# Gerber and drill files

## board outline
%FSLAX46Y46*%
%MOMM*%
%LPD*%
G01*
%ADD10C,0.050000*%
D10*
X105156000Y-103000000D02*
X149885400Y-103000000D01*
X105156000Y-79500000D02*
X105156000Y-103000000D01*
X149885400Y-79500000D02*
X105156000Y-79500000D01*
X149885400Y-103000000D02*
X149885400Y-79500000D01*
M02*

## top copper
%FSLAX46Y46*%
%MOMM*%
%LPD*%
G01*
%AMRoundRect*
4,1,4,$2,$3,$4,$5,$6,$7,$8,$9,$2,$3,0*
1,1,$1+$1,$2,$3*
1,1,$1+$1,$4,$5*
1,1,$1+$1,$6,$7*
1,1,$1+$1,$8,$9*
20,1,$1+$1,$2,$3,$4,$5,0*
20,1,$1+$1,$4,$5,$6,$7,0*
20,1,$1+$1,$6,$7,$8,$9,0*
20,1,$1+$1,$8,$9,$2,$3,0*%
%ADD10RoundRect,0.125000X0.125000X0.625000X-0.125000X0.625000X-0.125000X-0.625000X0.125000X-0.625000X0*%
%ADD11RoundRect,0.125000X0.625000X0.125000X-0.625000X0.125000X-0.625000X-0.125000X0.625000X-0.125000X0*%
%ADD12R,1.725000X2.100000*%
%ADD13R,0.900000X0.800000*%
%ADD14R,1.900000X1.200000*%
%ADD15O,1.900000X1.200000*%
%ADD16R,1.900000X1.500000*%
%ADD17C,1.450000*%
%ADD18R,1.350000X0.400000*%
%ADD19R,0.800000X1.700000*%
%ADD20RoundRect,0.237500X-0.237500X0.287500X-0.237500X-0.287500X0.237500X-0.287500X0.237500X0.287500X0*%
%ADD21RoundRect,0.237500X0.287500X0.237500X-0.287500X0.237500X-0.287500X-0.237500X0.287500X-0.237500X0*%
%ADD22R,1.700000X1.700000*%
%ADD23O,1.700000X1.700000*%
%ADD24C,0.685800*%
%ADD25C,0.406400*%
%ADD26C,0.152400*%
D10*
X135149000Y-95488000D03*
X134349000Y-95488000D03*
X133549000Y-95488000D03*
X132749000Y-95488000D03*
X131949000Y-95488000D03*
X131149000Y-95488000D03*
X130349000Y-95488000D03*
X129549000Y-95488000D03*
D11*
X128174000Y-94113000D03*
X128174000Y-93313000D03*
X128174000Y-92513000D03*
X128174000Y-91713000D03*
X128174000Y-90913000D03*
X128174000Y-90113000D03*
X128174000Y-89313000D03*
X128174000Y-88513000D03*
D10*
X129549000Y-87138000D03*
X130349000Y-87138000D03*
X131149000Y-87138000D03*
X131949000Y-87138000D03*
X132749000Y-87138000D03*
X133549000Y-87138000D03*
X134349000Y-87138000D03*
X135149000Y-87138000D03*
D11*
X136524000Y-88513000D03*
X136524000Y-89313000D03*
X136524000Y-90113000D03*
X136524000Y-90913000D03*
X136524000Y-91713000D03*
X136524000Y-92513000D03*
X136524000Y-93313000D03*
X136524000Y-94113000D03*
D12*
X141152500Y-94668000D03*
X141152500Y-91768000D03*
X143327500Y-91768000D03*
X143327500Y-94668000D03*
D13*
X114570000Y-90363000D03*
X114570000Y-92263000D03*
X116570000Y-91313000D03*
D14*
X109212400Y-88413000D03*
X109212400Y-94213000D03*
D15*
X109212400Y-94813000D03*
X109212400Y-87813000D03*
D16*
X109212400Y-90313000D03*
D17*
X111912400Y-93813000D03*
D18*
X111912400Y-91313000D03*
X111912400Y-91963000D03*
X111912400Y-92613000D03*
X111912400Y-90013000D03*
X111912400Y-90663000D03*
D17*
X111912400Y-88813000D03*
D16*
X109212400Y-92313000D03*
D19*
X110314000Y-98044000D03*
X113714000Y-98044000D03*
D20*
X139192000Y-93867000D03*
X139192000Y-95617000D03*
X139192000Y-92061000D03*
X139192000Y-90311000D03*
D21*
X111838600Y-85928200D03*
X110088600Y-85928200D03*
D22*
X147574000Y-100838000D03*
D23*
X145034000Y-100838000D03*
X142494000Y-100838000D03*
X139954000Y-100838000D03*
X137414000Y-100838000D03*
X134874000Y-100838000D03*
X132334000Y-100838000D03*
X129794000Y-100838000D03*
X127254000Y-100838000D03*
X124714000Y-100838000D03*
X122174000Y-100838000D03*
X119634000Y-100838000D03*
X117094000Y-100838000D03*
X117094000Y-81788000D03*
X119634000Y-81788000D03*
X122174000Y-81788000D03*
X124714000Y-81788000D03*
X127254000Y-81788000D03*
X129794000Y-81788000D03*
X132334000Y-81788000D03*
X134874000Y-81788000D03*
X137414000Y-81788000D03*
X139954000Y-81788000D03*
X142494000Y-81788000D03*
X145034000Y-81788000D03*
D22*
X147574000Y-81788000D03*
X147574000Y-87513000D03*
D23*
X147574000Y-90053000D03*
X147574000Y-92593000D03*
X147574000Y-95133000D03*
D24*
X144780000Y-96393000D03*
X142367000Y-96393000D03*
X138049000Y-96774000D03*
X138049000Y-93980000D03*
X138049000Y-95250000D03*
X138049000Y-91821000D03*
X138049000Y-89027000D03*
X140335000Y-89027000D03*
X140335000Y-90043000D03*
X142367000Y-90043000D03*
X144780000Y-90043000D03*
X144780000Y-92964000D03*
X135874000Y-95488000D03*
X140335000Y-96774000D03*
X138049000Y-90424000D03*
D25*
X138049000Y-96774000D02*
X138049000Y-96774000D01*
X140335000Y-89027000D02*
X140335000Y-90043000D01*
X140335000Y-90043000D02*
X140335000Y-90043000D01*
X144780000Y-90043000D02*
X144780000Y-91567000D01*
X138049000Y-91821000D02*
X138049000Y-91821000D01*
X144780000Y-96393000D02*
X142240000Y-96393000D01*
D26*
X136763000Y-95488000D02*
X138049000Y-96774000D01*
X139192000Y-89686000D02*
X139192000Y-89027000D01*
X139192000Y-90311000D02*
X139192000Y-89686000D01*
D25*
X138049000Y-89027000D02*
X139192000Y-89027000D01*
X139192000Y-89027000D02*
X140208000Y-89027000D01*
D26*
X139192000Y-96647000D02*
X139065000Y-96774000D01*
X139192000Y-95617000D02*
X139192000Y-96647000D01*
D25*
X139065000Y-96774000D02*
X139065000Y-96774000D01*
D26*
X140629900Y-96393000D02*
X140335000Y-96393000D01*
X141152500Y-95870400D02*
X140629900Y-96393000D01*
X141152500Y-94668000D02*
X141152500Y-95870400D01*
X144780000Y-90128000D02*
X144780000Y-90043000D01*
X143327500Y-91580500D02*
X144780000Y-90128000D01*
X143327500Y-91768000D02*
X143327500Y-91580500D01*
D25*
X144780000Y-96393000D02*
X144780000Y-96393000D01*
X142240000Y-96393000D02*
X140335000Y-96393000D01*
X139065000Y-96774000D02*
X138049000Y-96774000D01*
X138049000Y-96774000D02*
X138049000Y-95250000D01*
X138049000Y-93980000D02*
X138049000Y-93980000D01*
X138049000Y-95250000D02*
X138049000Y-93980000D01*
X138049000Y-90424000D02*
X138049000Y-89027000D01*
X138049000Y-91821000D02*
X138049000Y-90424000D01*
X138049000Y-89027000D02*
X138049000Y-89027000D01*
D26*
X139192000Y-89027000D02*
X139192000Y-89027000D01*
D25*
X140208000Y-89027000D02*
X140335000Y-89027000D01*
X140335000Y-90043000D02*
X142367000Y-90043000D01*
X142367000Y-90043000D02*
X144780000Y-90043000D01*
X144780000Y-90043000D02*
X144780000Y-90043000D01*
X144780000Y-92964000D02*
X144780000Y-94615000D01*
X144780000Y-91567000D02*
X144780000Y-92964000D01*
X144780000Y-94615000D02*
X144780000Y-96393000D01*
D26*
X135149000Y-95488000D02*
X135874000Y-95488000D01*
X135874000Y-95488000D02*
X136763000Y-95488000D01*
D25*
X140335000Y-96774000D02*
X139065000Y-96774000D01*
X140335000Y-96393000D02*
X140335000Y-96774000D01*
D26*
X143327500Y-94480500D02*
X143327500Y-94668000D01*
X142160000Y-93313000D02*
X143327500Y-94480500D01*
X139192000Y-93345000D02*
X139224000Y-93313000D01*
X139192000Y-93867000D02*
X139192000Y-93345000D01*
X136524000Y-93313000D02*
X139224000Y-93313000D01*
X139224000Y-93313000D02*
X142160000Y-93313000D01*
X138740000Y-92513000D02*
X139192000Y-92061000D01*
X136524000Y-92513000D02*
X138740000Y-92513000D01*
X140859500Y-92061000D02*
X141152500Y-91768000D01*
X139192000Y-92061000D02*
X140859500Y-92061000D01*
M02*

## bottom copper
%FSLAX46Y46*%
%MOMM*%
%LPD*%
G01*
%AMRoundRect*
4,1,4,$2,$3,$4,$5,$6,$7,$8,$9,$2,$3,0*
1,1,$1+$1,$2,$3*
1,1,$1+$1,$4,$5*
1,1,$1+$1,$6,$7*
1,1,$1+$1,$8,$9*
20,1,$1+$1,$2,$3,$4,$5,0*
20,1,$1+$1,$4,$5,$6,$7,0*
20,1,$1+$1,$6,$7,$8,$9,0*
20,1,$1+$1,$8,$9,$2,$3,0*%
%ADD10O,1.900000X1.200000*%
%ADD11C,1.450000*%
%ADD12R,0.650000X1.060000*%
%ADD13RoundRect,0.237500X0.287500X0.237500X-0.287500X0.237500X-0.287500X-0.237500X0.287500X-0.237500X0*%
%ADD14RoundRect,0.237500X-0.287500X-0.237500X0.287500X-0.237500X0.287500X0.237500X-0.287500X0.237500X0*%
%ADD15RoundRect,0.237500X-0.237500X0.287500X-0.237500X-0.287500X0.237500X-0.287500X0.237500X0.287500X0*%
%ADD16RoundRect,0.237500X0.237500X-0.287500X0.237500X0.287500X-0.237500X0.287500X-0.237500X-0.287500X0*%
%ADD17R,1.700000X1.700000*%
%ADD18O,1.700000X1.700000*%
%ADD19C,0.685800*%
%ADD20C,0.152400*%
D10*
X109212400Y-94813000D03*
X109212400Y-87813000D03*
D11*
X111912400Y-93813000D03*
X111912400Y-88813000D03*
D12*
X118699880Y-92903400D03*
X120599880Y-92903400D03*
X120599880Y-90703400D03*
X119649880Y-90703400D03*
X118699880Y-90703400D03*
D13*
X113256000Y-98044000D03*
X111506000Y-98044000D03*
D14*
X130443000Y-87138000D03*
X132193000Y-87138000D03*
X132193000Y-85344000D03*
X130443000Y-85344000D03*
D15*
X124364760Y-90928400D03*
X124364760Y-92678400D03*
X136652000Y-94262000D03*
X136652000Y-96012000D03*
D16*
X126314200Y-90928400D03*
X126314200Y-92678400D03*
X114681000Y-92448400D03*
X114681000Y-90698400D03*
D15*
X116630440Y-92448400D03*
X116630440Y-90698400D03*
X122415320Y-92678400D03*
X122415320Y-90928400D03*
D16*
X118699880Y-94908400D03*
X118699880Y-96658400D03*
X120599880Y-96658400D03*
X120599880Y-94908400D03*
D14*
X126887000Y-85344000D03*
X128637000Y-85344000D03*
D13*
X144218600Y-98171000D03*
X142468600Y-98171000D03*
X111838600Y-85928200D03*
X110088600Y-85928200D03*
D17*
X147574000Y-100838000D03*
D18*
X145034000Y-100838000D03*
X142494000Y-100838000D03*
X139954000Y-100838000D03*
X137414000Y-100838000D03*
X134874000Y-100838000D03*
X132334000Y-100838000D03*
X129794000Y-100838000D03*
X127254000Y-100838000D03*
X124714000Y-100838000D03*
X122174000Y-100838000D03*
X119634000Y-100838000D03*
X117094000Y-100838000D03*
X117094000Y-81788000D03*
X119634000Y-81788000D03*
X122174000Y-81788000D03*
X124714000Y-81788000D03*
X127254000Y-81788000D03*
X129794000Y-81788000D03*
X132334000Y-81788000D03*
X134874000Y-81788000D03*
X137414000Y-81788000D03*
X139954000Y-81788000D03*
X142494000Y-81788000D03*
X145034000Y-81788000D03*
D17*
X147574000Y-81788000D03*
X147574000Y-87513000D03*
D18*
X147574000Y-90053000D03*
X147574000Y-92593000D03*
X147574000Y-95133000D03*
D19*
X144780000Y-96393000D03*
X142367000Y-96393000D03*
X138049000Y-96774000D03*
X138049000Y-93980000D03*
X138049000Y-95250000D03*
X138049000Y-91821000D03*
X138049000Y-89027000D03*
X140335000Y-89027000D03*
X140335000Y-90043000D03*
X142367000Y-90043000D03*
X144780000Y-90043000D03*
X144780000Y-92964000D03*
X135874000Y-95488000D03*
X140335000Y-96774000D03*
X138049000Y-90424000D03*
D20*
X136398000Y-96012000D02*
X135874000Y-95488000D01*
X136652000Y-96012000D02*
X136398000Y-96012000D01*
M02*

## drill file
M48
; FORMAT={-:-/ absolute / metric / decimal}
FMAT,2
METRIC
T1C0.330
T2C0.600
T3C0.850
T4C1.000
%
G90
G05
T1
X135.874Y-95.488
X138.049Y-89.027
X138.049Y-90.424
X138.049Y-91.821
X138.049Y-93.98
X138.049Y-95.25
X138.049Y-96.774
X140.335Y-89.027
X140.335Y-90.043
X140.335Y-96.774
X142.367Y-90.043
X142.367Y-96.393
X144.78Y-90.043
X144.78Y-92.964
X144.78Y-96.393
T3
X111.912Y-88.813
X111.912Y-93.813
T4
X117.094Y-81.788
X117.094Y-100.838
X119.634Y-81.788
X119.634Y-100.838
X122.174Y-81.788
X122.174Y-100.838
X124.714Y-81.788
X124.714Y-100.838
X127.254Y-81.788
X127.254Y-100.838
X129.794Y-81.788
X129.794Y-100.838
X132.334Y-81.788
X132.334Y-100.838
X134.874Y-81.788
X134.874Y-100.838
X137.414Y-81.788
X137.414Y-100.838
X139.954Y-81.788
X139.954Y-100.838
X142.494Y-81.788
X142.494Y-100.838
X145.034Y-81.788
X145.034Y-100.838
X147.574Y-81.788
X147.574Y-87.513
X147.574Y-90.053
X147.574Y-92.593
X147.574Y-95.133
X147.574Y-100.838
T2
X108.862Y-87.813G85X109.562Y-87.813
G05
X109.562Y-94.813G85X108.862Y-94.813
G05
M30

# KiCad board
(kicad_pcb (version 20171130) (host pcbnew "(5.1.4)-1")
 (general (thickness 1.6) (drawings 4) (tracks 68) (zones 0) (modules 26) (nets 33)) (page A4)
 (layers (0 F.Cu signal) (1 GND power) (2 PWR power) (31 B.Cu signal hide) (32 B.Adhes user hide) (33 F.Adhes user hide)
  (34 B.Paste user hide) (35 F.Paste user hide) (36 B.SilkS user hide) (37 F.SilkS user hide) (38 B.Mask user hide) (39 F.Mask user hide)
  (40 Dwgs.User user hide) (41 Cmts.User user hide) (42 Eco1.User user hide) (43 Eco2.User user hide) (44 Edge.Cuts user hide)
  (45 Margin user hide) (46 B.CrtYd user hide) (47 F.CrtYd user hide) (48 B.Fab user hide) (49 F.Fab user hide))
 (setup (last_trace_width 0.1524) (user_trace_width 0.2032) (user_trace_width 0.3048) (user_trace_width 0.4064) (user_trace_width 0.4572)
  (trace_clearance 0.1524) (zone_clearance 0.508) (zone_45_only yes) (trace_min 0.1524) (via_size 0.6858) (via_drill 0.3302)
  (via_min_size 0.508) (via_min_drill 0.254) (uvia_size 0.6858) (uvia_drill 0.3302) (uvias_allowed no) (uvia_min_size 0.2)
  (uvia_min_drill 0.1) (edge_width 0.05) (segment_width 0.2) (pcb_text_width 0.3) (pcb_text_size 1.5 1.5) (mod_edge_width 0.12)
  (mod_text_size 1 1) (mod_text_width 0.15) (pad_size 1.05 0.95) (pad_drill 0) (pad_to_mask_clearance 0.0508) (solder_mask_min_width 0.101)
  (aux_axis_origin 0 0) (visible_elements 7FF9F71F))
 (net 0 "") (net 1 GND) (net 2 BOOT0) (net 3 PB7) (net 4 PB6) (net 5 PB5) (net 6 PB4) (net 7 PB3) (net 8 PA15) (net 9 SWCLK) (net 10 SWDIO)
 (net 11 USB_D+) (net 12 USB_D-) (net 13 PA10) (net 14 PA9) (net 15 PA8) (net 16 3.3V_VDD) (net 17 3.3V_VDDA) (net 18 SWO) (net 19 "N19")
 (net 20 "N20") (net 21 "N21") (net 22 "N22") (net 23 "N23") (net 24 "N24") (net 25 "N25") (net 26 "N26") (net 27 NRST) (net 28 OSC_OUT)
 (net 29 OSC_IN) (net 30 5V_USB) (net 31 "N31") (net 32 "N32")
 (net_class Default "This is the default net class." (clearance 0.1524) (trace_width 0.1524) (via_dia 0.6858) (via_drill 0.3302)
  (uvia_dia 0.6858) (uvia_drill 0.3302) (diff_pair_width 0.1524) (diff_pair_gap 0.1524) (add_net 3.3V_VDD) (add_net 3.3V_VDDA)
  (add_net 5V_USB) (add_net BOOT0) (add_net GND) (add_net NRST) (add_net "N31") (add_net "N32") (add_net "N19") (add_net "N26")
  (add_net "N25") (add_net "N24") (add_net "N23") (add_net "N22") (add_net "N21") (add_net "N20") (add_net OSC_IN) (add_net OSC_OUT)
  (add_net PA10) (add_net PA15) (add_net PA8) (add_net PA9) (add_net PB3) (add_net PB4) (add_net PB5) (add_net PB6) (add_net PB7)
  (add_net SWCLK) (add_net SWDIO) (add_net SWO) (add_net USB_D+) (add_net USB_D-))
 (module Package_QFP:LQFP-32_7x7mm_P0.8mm (layer F.Cu) (at 132.349 91.313 180)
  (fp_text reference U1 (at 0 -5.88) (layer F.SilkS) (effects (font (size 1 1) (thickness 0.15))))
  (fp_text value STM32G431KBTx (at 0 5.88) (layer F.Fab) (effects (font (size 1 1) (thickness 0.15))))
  (pad 32 smd roundrect (at -2.8 -4.175 180) (size 0.5 1.5) (layers F.Cu F.Paste F.Mask) (roundrect_rratio 0.25) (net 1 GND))
  (pad 31 smd roundrect (at -2 -4.175 180) (size 0.5 1.5) (layers F.Cu F.Paste F.Mask) (roundrect_rratio 0.25) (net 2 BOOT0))
  (pad 30 smd roundrect (at -1.2 -4.175 180) (size 0.5 1.5) (layers F.Cu F.Paste F.Mask) (roundrect_rratio 0.25) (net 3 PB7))
  (pad 29 smd roundrect (at -0.4 -4.175 180) (size 0.5 1.5) (layers F.Cu F.Paste F.Mask) (roundrect_rratio 0.25) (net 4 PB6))
  (pad 28 smd roundrect (at 0.4 -4.175 180) (size 0.5 1.5) (layers F.Cu F.Paste F.Mask) (roundrect_rratio 0.25) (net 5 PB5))
  (pad 27 smd roundrect (at 1.2 -4.175 180) (size 0.5 1.5) (layers F.Cu F.Paste F.Mask) (roundrect_rratio 0.25) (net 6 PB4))
  (pad 26 smd roundrect (at 2 -4.175 180) (size 0.5 1.5) (layers F.Cu F.Paste F.Mask) (roundrect_rratio 0.25) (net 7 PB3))
  (pad 25 smd roundrect (at 2.8 -4.175 180) (size 0.5 1.5) (layers F.Cu F.Paste F.Mask) (roundrect_rratio 0.25) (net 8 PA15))
  (pad 24 smd roundrect (at 4.175 -2.8 180) (size 1.5 0.5) (layers F.Cu F.Paste F.Mask) (roundrect_rratio 0.25) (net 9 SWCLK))
  (pad 23 smd roundrect (at 4.175 -2 180) (size 1.5 0.5) (layers F.Cu F.Paste F.Mask) (roundrect_rratio 0.25) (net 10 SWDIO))
  (pad 22 smd roundrect (at 4.175 -1.2 180) (size 1.5 0.5) (layers F.Cu F.Paste F.Mask) (roundrect_rratio 0.25) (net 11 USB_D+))
  (pad 21 smd roundrect (at 4.175 -0.4 180) (size 1.5 0.5) (layers F.Cu F.Paste F.Mask) (roundrect_rratio 0.25) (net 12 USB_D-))
  (pad 20 smd roundrect (at 4.175 0.4 180) (size 1.5 0.5) (layers F.Cu F.Paste F.Mask) (roundrect_rratio 0.25) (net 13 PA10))
  (pad 19 smd roundrect (at 4.175 1.2 180) (size 1.5 0.5) (layers F.Cu F.Paste F.Mask) (roundrect_rratio 0.25) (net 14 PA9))
  (pad 18 smd roundrect (at 4.175 2 180) (size 1.5 0.5) (layers F.Cu F.Paste F.Mask) (roundrect_rratio 0.25) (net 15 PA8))
  (pad 17 smd roundrect (at 4.175 2.8 180) (size 1.5 0.5) (layers F.Cu F.Paste F.Mask) (roundrect_rratio 0.25) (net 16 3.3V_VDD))
  (pad 16 smd roundrect (at 2.8 4.175 180) (size 0.5 1.5) (layers F.Cu F.Paste F.Mask) (roundrect_rratio 0.25) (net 1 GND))
  (pad 15 smd roundrect (at 2 4.175 180) (size 0.5 1.5) (layers F.Cu F.Paste F.Mask) (roundrect_rratio 0.25) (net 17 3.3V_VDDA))
  (pad 14 smd roundrect (at 1.2 4.175 180) (size 0.5 1.5) (layers F.Cu F.Paste F.Mask) (roundrect_rratio 0.25) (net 1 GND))
  (pad 13 smd roundrect (at 0.4 4.175 180) (size 0.5 1.5) (layers F.Cu F.Paste F.Mask) (roundrect_rratio 0.25) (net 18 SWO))
  (pad 12 smd roundrect (at -0.4 4.175 180) (size 0.5 1.5) (layers F.Cu F.Paste F.Mask) (roundrect_rratio 0.25) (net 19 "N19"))
  (pad 11 smd roundrect (at -1.2 4.175 180) (size 0.5 1.5) (layers F.Cu F.Paste F.Mask) (roundrect_rratio 0.25) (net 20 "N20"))
  (pad 10 smd roundrect (at -2 4.175 180) (size 0.5 1.5) (layers F.Cu F.Paste F.Mask) (roundrect_rratio 0.25) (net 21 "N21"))
  (pad 9 smd roundrect (at -2.8 4.175 180) (size 0.5 1.5) (layers F.Cu F.Paste F.Mask) (roundrect_rratio 0.25) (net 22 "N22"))
  (pad 8 smd roundrect (at -4.175 2.8 180) (size 1.5 0.5) (layers F.Cu F.Paste F.Mask) (roundrect_rratio 0.25) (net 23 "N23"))
  (pad 7 smd roundrect (at -4.175 2 180) (size 1.5 0.5) (layers F.Cu F.Paste F.Mask) (roundrect_rratio 0.25) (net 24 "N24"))
  (pad 6 smd roundrect (at -4.175 1.2 180) (size 1.5 0.5) (layers F.Cu F.Paste F.Mask) (roundrect_rratio 0.25) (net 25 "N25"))
  (pad 5 smd roundrect (at -4.175 0.4 180) (size 1.5 0.5) (layers F.Cu F.Paste F.Mask) (roundrect_rratio 0.25) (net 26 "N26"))
  (pad 4 smd roundrect (at -4.175 -0.4 180) (size 1.5 0.5) (layers F.Cu F.Paste F.Mask) (roundrect_rratio 0.25) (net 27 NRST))
  (pad 3 smd roundrect (at -4.175 -1.2 180) (size 1.5 0.5) (layers F.Cu F.Paste F.Mask) (roundrect_rratio 0.25) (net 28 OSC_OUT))
  (pad 2 smd roundrect (at -4.175 -2 180) (size 1.5 0.5) (layers F.Cu F.Paste F.Mask) (roundrect_rratio 0.25) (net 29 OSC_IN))
  (pad 1 smd roundrect (at -4.175 -2.8 180) (size 1.5 0.5) (layers F.Cu F.Paste F.Mask) (roundrect_rratio 0.25) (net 16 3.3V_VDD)))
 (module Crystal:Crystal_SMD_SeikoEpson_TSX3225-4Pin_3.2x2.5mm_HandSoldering (layer F.Cu) (at 142.24 93.218 90)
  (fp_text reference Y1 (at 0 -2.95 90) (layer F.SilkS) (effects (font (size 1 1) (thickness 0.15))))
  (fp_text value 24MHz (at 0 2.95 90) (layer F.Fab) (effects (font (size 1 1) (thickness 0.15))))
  (pad 4 smd rect (at -1.45 -1.0875 90) (size 2.1 1.725) (layers F.Cu F.Paste F.Mask) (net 1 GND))
  (pad 3 smd rect (at 1.45 -1.0875 90) (size 2.1 1.725) (layers F.Cu F.Paste F.Mask) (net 28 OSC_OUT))
  (pad 2 smd rect (at 1.45 1.0875 90) (size 2.1 1.725) (layers F.Cu F.Paste F.Mask) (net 1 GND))
  (pad 1 smd rect (at -1.45 1.0875 90) (size 2.1 1.725) (layers F.Cu F.Paste F.Mask) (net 29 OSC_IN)))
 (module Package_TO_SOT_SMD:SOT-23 (layer F.Cu) (at 115.57 91.313)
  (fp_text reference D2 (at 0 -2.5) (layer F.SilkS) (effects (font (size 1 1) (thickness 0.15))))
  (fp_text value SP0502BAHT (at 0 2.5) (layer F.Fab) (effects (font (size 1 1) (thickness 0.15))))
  (pad 1 smd rect (at -1 -0.95) (size 0.9 0.8) (layers F.Cu F.Paste F.Mask) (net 12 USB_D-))
  (pad 2 smd rect (at -1 0.95) (size 0.9 0.8) (layers F.Cu F.Paste F.Mask) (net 11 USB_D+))
  (pad 3 smd rect (at 1 0) (size 0.9 0.8) (layers F.Cu F.Paste F.Mask) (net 1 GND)))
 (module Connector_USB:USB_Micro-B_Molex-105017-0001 (layer F.Cu) (at 110.4499 91.313 270)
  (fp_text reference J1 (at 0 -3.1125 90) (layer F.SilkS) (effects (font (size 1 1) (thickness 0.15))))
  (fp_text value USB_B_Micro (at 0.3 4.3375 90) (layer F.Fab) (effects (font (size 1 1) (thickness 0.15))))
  (pad 6 smd rect (at -2.9 1.2375 270) (size 1.2 1.9) (layers F.Cu F.Mask) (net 1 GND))
  (pad 6 smd rect (at 2.9 1.2375 270) (size 1.2 1.9) (layers F.Cu F.Mask) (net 1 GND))
  (pad 6 thru_hole oval (at 3.5 1.2375 270) (size 1.2 1.9) (drill oval 0.6 1.3) (layers *.Cu *.Mask) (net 1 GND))
  (pad 6 thru_hole oval (at -3.5 1.2375 90) (size 1.2 1.9) (drill oval 0.6 1.3) (layers *.Cu *.Mask) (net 1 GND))
  (pad 6 smd rect (at -1 1.2375 270) (size 1.5 1.9) (layers F.Cu F.Paste F.Mask) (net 1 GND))
  (pad 6 thru_hole circle (at 2.5 -1.4625 270) (size 1.45 1.45) (drill 0.85) (layers *.Cu *.Mask) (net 1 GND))
  (pad 3 smd rect (at 0 -1.4625 270) (size 0.4 1.35) (layers F.Cu F.Paste F.Mask) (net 11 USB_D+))
  (pad 4 smd rect (at 0.65 -1.4625 270) (size 0.4 1.35) (layers F.Cu F.Paste F.Mask))
  (pad 5 smd rect (at 1.3 -1.4625 270) (size 0.4 1.35) (layers F.Cu F.Paste F.Mask) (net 1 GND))
  (pad 1 smd rect (at -1.3 -1.4625 270) (size 0.4 1.35) (layers F.Cu F.Paste F.Mask) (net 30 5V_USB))
  (pad 2 smd rect (at -0.65 -1.4625 270) (size 0.4 1.35) (layers F.Cu F.Paste F.Mask) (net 12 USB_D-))
  (pad 6 thru_hole circle (at -2.5 -1.4625 270) (size 1.45 1.45) (drill 0.85) (layers *.Cu *.Mask) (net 1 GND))
  (pad 6 smd rect (at 1 1.2375 270) (size 1.5 1.9) (layers F.Cu F.Paste F.Mask) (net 1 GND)))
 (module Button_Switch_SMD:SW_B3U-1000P (layer F.Cu) (at 112.014 98.044 180)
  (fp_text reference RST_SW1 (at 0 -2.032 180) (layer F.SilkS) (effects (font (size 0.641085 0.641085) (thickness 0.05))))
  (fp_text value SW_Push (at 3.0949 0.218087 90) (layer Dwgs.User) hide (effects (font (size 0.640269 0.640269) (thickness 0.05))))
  (pad 1 smd rect (at 1.7 0 180) (size 0.8 1.7) (layers F.Cu F.Paste F.Mask) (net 1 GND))
  (pad 2 smd rect (at -1.7 0 180) (size 0.8 1.7) (layers F.Cu F.Paste F.Mask) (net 27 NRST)))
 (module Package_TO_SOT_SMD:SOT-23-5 (layer B.Cu) (at 119.64988 91.8034 270)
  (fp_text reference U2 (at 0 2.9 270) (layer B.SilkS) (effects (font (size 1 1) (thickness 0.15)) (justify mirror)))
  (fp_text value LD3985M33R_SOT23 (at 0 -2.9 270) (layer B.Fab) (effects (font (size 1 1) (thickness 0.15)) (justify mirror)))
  (pad 5 smd rect (at 1.1 0.95 270) (size 1.06 0.65) (layers B.Cu B.Paste B.Mask) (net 16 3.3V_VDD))
  (pad 4 smd rect (at 1.1 -0.95 270) (size 1.06 0.65) (layers B.Cu B.Paste B.Mask) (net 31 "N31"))
  (pad 3 smd rect (at -1.1 -0.95 270) (size 1.06 0.65) (layers B.Cu B.Paste B.Mask) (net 30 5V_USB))
  (pad 2 smd rect (at -1.1 0 270) (size 1.06 0.65) (layers B.Cu B.Paste B.Mask) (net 1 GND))
  (pad 1 smd rect (at -1.1 0.95 270) (size 1.06 0.65) (layers B.Cu B.Paste B.Mask) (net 30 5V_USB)))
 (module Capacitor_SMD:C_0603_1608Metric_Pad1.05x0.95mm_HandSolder (layer B.Cu) (at 112.381 98.044 180)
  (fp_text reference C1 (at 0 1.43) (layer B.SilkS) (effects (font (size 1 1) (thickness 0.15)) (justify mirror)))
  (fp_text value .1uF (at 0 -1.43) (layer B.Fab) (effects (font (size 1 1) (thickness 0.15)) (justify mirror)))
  (pad 1 smd roundrect (at -0.875 0 180) (size 1.05 0.95) (layers B.Cu B.Paste B.Mask) (roundrect_rratio 0.25) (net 27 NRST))
  (pad 2 smd roundrect (at 0.875 0 180) (size 1.05 0.95) (layers B.Cu B.Paste B.Mask) (roundrect_rratio 0.25) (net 1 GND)))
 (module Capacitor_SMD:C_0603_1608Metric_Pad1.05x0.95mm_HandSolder (layer F.Cu) (at 139.192 94.742 270)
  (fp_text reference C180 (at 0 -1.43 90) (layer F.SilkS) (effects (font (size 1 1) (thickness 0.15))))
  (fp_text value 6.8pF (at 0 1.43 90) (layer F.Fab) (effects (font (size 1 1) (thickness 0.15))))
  (pad 1 smd roundrect (at -0.875 0 270) (size 1.05 0.95) (layers F.Cu F.Paste F.Mask) (roundrect_rratio 0.25) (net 29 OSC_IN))
  (pad 2 smd roundrect (at 0.875 0 270) (size 1.05 0.95) (layers F.Cu F.Paste F.Mask) (roundrect_rratio 0.25) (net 1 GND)))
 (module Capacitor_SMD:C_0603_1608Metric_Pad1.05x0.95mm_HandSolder (layer F.Cu) (at 139.192 91.186 270)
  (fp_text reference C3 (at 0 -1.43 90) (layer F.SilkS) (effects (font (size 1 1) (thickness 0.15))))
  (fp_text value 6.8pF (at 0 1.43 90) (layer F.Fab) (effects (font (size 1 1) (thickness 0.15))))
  (pad 2 smd roundrect (at 0.875 0 270) (size 1.05 0.95) (layers F.Cu F.Paste F.Mask) (roundrect_rratio 0.25) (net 28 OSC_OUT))
  (pad 1 smd roundrect (at -0.875 0 270) (size 1.05 0.95) (layers F.Cu F.Paste F.Mask) (roundrect_rratio 0.25) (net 1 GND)))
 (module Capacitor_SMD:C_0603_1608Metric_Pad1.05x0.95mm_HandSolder (layer B.Cu) (at 131.318 87.138)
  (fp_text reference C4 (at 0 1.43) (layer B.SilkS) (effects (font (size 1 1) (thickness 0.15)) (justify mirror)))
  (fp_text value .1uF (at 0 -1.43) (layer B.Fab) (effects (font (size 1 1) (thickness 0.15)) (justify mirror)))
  (pad 1 smd roundrect (at -0.875 0) (size 1.05 0.95) (layers B.Cu B.Paste B.Mask) (roundrect_rratio 0.25) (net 17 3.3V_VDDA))
  (pad 2 smd roundrect (at 0.875 0) (size 1.05 0.95) (layers B.Cu B.Paste B.Mask) (roundrect_rratio 0.25) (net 1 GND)))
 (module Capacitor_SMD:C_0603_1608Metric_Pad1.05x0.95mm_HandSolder (layer B.Cu) (at 131.318 85.344)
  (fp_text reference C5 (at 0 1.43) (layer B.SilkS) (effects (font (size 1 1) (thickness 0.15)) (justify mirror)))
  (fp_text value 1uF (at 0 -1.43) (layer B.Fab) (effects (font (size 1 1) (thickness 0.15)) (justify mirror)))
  (pad 2 smd roundrect (at 0.875 0) (size 1.05 0.95) (layers B.Cu B.Paste B.Mask) (roundrect_rratio 0.25) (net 1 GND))
  (pad 1 smd roundrect (at -0.875 0) (size 1.05 0.95) (layers B.Cu B.Paste B.Mask) (roundrect_rratio 0.25) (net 17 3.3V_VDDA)))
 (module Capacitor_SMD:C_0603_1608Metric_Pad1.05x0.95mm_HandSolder (layer B.Cu) (at 124.36476 91.8034 270)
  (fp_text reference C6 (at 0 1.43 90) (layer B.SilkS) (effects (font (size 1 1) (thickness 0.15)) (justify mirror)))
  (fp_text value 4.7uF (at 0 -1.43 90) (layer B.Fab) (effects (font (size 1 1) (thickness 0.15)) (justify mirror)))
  (pad 1 smd roundrect (at -0.875 0 270) (size 1.05 0.95) (layers B.Cu B.Paste B.Mask) (roundrect_rratio 0.25) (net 1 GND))
  (pad 2 smd roundrect (at 0.875 0 270) (size 1.05 0.95) (layers B.Cu B.Paste B.Mask) (roundrect_rratio 0.25) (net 16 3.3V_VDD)))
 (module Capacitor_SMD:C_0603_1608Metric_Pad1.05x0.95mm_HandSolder (layer B.Cu) (at 136.652 95.137 270)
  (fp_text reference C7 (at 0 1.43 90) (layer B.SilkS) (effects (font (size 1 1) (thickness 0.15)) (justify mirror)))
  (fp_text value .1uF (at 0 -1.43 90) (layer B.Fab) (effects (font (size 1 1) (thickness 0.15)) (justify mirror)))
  (pad 1 smd roundrect (at -0.875 0 270) (size 1.05 0.95) (layers B.Cu B.Paste B.Mask) (roundrect_rratio 0.25) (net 16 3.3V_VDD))
  (pad 2 smd roundrect (at 0.875 0 270) (size 1.05 0.95) (layers B.Cu B.Paste B.Mask) (roundrect_rratio 0.25) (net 1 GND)))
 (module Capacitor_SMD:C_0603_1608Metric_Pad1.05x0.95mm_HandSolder (layer B.Cu) (at 126.3142 91.8034 90)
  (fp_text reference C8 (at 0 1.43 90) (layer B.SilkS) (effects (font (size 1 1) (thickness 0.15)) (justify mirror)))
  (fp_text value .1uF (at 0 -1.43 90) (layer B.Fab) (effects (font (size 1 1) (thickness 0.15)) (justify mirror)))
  (pad 2 smd roundrect (at 0.875 0 90) (size 1.05 0.95) (layers B.Cu B.Paste B.Mask) (roundrect_rratio 0.25) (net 1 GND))
  (pad 1 smd roundrect (at -0.875 0 90) (size 1.05 0.95) (layers B.Cu B.Paste B.Mask) (roundrect_rratio 0.25) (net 16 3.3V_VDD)))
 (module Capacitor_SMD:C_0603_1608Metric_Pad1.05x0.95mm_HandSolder (layer B.Cu) (at 114.681 91.5734 90)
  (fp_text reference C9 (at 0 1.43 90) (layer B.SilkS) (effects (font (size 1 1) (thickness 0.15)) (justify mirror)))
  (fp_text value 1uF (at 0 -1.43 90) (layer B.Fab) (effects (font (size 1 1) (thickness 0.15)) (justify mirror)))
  (pad 1 smd roundrect (at -0.875 0 90) (size 1.05 0.95) (layers B.Cu B.Paste B.Mask) (roundrect_rratio 0.25) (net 1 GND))
  (pad 2 smd roundrect (at 0.875 0 90) (size 1.05 0.95) (layers B.Cu B.Paste B.Mask) (roundrect_rratio 0.25) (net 30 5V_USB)))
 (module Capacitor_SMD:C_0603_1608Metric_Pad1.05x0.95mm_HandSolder (layer B.Cu) (at 116.63044 91.5734 270)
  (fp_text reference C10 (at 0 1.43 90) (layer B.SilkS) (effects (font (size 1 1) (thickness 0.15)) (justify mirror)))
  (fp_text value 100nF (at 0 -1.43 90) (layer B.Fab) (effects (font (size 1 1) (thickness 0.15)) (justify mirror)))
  (pad 2 smd roundrect (at 0.875 0 270) (size 1.05 0.95) (layers B.Cu B.Paste B.Mask) (roundrect_rratio 0.25) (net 1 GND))
  (pad 1 smd roundrect (at -0.875 0 270) (size 1.05 0.95) (layers B.Cu B.Paste B.Mask) (roundrect_rratio 0.25) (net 30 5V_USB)))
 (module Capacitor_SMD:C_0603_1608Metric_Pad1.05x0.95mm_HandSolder (layer B.Cu) (at 122.41532 91.8034 270)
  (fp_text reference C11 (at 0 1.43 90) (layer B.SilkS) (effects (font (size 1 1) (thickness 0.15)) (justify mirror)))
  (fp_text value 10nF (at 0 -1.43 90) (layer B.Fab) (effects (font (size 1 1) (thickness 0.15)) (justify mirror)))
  (pad 2 smd roundrect (at 0.875 0 270) (size 1.05 0.95) (layers B.Cu B.Paste B.Mask) (roundrect_rratio 0.25) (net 31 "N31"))
  (pad 1 smd roundrect (at -0.875 0 270) (size 1.05 0.95) (layers B.Cu B.Paste B.Mask) (roundrect_rratio 0.25) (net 1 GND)))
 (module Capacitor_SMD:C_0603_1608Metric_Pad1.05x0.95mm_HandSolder (layer B.Cu) (at 118.69988 95.7834 90)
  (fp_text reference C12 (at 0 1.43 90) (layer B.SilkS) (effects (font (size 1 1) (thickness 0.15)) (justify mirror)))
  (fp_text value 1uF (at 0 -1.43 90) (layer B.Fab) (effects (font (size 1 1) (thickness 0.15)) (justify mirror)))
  (pad 2 smd roundrect (at 0.875 0 90) (size 1.05 0.95) (layers B.Cu B.Paste B.Mask) (roundrect_rratio 0.25) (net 16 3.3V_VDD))
  (pad 1 smd roundrect (at -0.875 0 90) (size 1.05 0.95) (layers B.Cu B.Paste B.Mask) (roundrect_rratio 0.25) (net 1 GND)))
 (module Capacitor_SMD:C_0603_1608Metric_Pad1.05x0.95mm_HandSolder (layer B.Cu) (at 120.59988 95.7834 90)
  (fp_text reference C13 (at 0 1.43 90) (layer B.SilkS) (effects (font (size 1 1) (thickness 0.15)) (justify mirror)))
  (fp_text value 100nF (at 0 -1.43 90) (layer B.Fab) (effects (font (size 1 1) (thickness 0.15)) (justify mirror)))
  (pad 1 smd roundrect (at -0.875 0 90) (size 1.05 0.95) (layers B.Cu B.Paste B.Mask) (roundrect_rratio 0.25) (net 1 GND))
  (pad 2 smd roundrect (at 0.875 0 90) (size 1.05 0.95) (layers B.Cu B.Paste B.Mask) (roundrect_rratio 0.25) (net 16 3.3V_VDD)))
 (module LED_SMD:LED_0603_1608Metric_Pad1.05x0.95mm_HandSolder (layer F.Cu) (at 110.9636 85.9282 180)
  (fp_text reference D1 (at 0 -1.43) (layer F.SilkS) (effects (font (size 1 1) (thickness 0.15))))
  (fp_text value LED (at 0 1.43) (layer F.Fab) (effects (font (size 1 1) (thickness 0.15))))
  (pad 1 smd roundrect (at -0.875 0 180) (size 1.05 0.95) (layers F.Cu F.Paste F.Mask) (roundrect_rratio 0.25) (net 1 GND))
  (pad 2 smd roundrect (at 0.875 0 180) (size 1.05 0.95) (layers F.Cu F.Paste F.Mask) (roundrect_rratio 0.25) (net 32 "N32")))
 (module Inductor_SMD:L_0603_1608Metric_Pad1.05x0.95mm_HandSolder (layer B.Cu) (at 127.762 85.344)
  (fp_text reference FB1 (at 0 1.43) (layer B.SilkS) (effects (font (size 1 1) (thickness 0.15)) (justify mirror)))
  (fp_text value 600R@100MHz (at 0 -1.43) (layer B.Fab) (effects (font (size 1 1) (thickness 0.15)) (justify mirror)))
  (pad 1 smd roundrect (at -0.875 0) (size 1.05 0.95) (layers B.Cu B.Paste B.Mask) (roundrect_rratio 0.25) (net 16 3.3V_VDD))
  (pad 2 smd roundrect (at 0.875 0) (size 1.05 0.95) (layers B.Cu B.Paste B.Mask) (roundrect_rratio 0.25) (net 17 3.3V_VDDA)))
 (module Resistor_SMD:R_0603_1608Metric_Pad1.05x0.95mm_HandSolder (layer B.Cu) (at 143.3436 98.171 180)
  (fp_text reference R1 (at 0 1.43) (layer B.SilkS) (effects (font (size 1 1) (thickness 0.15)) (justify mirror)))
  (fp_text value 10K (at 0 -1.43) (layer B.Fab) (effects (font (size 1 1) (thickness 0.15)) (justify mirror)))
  (pad 1 smd roundrect (at -0.875 0 180) (size 1.05 0.95) (layers B.Cu B.Paste B.Mask) (roundrect_rratio 0.25) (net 1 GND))
  (pad 2 smd roundrect (at 0.875 0 180) (size 1.05 0.95) (layers B.Cu B.Paste B.Mask) (roundrect_rratio 0.25) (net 2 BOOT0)))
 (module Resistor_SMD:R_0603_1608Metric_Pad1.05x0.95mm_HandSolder (layer B.Cu) (at 110.9636 85.9282 180)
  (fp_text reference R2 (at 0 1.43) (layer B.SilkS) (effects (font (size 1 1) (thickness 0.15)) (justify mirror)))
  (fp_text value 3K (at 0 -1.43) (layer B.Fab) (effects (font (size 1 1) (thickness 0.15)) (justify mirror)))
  (pad 1 smd roundrect (at -0.875 0 180) (size 1.05 0.95) (layers B.Cu B.Paste B.Mask) (roundrect_rratio 0.25) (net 30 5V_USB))
  (pad 2 smd roundrect (at 0.875 0 180) (size 1.05 0.95) (layers B.Cu B.Paste B.Mask) (roundrect_rratio 0.25) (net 32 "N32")))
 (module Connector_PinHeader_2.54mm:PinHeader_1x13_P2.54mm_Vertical (layer F.Cu) (at 147.574 100.838 270)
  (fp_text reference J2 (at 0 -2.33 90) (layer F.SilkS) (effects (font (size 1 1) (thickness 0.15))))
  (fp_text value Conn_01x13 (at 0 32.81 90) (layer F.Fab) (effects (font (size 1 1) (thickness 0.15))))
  (pad 1 thru_hole rect (at 0 0 270) (size 1.7 1.7) (drill 1) (layers *.Cu *.Mask) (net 16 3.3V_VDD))
  (pad 2 thru_hole oval (at 0 2.54 270) (size 1.7 1.7) (drill 1) (layers *.Cu *.Mask) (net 1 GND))
  (pad 3 thru_hole oval (at 0 5.08 270) (size 1.7 1.7) (drill 1) (layers *.Cu *.Mask) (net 2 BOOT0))
  (pad 4 thru_hole oval (at 0 7.62 270) (size 1.7 1.7) (drill 1) (layers *.Cu *.Mask) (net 27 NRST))
  (pad 5 thru_hole oval (at 0 10.16 270) (size 1.7 1.7) (drill 1) (layers *.Cu *.Mask) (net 3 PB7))
  (pad 6 thru_hole oval (at 0 12.7 270) (size 1.7 1.7) (drill 1) (layers *.Cu *.Mask) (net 4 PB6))
  (pad 7 thru_hole oval (at 0 15.24 270) (size 1.7 1.7) (drill 1) (layers *.Cu *.Mask) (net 5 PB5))
  (pad 8 thru_hole oval (at 0 17.78 270) (size 1.7 1.7) (drill 1) (layers *.Cu *.Mask) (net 6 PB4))
  (pad 9 thru_hole oval (at 0 20.32 270) (size 1.7 1.7) (drill 1) (layers *.Cu *.Mask) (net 7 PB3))
  (pad 10 thru_hole oval (at 0 22.86 270) (size 1.7 1.7) (drill 1) (layers *.Cu *.Mask) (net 8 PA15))
  (pad 11 thru_hole oval (at 0 25.4 270) (size 1.7 1.7) (drill 1) (layers *.Cu *.Mask) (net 13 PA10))
  (pad 12 thru_hole oval (at 0 27.94 270) (size 1.7 1.7) (drill 1) (layers *.Cu *.Mask) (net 14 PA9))
  (pad 13 thru_hole oval (at 0 30.48 270) (size 1.7 1.7) (drill 1) (layers *.Cu *.Mask) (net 15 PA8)))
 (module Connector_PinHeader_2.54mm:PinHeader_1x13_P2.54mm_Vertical (layer F.Cu) (at 147.574 81.788 270)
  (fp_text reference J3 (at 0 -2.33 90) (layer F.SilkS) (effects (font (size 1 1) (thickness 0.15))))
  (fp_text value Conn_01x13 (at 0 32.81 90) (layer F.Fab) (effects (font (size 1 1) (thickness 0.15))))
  (pad 13 thru_hole oval (at 0 30.48 270) (size 1.7 1.7) (drill 1) (layers *.Cu *.Mask) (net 30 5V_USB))
  (pad 12 thru_hole oval (at 0 27.94 270) (size 1.7 1.7) (drill 1) (layers *.Cu *.Mask) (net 1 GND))
  (pad 11 thru_hole oval (at 0 25.4 270) (size 1.7 1.7) (drill 1) (layers *.Cu *.Mask) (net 18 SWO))
  (pad 10 thru_hole oval (at 0 22.86 270) (size 1.7 1.7) (drill 1) (layers *.Cu *.Mask) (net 19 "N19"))
  (pad 9 thru_hole oval (at 0 20.32 270) (size 1.7 1.7) (drill 1) (layers *.Cu *.Mask) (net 20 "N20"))
  (pad 8 thru_hole oval (at 0 17.78 270) (size 1.7 1.7) (drill 1) (layers *.Cu *.Mask) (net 21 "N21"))
  (pad 7 thru_hole oval (at 0 15.24 270) (size 1.7 1.7) (drill 1) (layers *.Cu *.Mask) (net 22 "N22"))
  (pad 6 thru_hole oval (at 0 12.7 270) (size 1.7 1.7) (drill 1) (layers *.Cu *.Mask) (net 23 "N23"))
  (pad 5 thru_hole oval (at 0 10.16 270) (size 1.7 1.7) (drill 1) (layers *.Cu *.Mask) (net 24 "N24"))
  (pad 4 thru_hole oval (at 0 7.62 270) (size 1.7 1.7) (drill 1) (layers *.Cu *.Mask) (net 25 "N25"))
  (pad 3 thru_hole oval (at 0 5.08 270) (size 1.7 1.7) (drill 1) (layers *.Cu *.Mask) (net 26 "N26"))
  (pad 2 thru_hole oval (at 0 2.54 270) (size 1.7 1.7) (drill 1) (layers *.Cu *.Mask) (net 1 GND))
  (pad 1 thru_hole rect (at 0 0 270) (size 1.7 1.7) (drill 1) (layers *.Cu *.Mask) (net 17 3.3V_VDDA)))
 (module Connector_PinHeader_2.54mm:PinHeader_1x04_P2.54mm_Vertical (layer F.Cu) (at 147.574 87.513)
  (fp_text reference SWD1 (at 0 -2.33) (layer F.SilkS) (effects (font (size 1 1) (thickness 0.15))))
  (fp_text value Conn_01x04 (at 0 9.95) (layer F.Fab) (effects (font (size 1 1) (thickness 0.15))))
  (pad 1 thru_hole rect (at 0 0) (size 1.7 1.7) (drill 1) (layers *.Cu *.Mask) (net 16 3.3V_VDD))
  (pad 2 thru_hole oval (at 0 2.54) (size 1.7 1.7) (drill 1) (layers *.Cu *.Mask) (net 10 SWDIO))
  (pad 3 thru_hole oval (at 0 5.08) (size 1.7 1.7) (drill 1) (layers *.Cu *.Mask) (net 9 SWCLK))
  (pad 4 thru_hole oval (at 0 7.62) (size 1.7 1.7) (drill 1) (layers *.Cu *.Mask) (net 1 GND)))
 (gr_line (start 105.156 103) (end 149.8854 103) (layer Edge.Cuts) (width 0.05))
 (gr_line (start 105.156 79.5) (end 105.156 103) (layer Edge.Cuts) (width 0.05))
 (gr_line (start 149.8854 79.5) (end 105.156 79.5) (layer Edge.Cuts) (width 0.05))
 (gr_line (start 149.8854 103) (end 149.8854 79.5) (layer Edge.Cuts) (width 0.05))
 (segment (start 138.049 96.774) (end 138.049 96.774) (width 0.4064) (layer F.Cu) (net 1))
 (segment (start 140.335 89.027) (end 140.335 90.043) (width 0.4064) (layer F.Cu) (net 1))
 (segment (start 140.335 90.043) (end 140.335 90.043) (width 0.4064) (layer F.Cu) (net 1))
 (segment (start 144.78 90.043) (end 144.78 91.567) (width 0.4064) (layer F.Cu) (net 1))
 (segment (start 138.049 91.821) (end 138.049 91.821) (width 0.4064) (layer F.Cu) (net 1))
 (segment (start 144.78 96.393) (end 142.24 96.393) (width 0.4064) (layer F.Cu) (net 1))
 (segment (start 136.763 95.488) (end 138.049 96.774) (width 0.1524) (layer F.Cu) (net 1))
 (segment (start 139.192 89.686) (end 139.192 89.027) (width 0.1524) (layer F.Cu) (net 1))
 (segment (start 139.192 90.311) (end 139.192 89.686) (width 0.1524) (layer F.Cu) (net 1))
 (segment (start 138.049 89.027) (end 139.192 89.027) (width 0.4064) (layer F.Cu) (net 1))
 (segment (start 139.192 89.027) (end 140.208 89.027) (width 0.4064) (layer F.Cu) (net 1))
 (segment (start 139.192 96.647) (end 139.065 96.774) (width 0.1524) (layer F.Cu) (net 1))
 (segment (start 139.192 95.617) (end 139.192 96.647) (width 0.1524) (layer F.Cu) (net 1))
 (segment (start 139.065 96.774) (end 139.065 96.774) (width 0.4064) (layer F.Cu) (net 1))
 (segment (start 140.6299 96.393) (end 140.335 96.393) (width 0.1524) (layer F.Cu) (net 1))
 (segment (start 141.1525 95.8704) (end 140.6299 96.393) (width 0.1524) (layer F.Cu) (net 1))
 (segment (start 141.1525 94.668) (end 141.1525 95.8704) (width 0.1524) (layer F.Cu) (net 1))
 (segment (start 144.78 90.128) (end 144.78 90.043) (width 0.1524) (layer F.Cu) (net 1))
 (segment (start 143.3275 91.5805) (end 144.78 90.128) (width 0.1524) (layer F.Cu) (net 1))
 (segment (start 143.3275 91.768) (end 143.3275 91.5805) (width 0.1524) (layer F.Cu) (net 1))
 (segment (start 144.78 96.393) (end 144.78 96.393) (width 0.4064) (layer F.Cu) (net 1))
 (via (at 144.78 96.393) (size 0.6858) (drill 0.3302) (layers F.Cu B.Cu) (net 1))
 (segment (start 142.24 96.393) (end 140.335 96.393) (width 0.4064) (layer F.Cu) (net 1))
 (via (at 142.367 96.393) (size 0.6858) (drill 0.3302) (layers F.Cu B.Cu) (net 1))
 (segment (start 139.065 96.774) (end 138.049 96.774) (width 0.4064) (layer F.Cu) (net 1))
 (segment (start 138.049 96.774) (end 138.049 95.25) (width 0.4064) (layer F.Cu) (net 1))
 (via (at 138.049 96.774) (size 0.6858) (drill 0.3302) (layers F.Cu B.Cu) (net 1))
 (segment (start 138.049 93.98) (end 138.049 93.98) (width 0.4064) (layer F.Cu) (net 1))
 (via (at 138.049 93.98) (size 0.6858) (drill 0.3302) (layers F.Cu B.Cu) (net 1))
 (segment (start 138.049 95.25) (end 138.049 93.98) (width 0.4064) (layer F.Cu) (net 1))
 (via (at 138.049 95.25) (size 0.6858) (drill 0.3302) (layers F.Cu B.Cu) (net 1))
 (segment (start 138.049 90.424) (end 138.049 89.027) (width 0.4064) (layer F.Cu) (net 1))
 (segment (start 138.049 91.821) (end 138.049 90.424) (width 0.4064) (layer F.Cu) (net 1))
 (via (at 138.049 91.821) (size 0.6858) (drill 0.3302) (layers F.Cu B.Cu) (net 1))
 (segment (start 138.049 89.027) (end 138.049 89.027) (width 0.4064) (layer F.Cu) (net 1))
 (via (at 138.049 89.027) (size 0.6858) (drill 0.3302) (layers F.Cu B.Cu) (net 1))
 (segment (start 139.192 89.027) (end 139.192 89.027) (width 0.1524) (layer F.Cu) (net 1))
 (segment (start 140.208 89.027) (end 140.335 89.027) (width 0.4064) (layer F.Cu) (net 1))
 (via (at 140.335 89.027) (size 0.6858) (drill 0.3302) (layers F.Cu B.Cu) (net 1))
 (segment (start 140.335 90.043) (end 142.367 90.043) (width 0.4064) (layer F.Cu) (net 1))
 (via (at 140.335 90.043) (size 0.6858) (drill 0.3302) (layers F.Cu B.Cu) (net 1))
 (segment (start 142.367 90.043) (end 144.78 90.043) (width 0.4064) (layer F.Cu) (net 1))
 (via (at 142.367 90.043) (size 0.6858) (drill 0.3302) (layers F.Cu B.Cu) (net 1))
 (segment (start 144.78 90.043) (end 144.78 90.043) (width 0.4064) (layer F.Cu) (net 1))
 (via (at 144.78 90.043) (size 0.6858) (drill 0.3302) (layers F.Cu B.Cu) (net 1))
 (segment (start 144.78 92.964) (end 144.78 94.615) (width 0.4064) (layer F.Cu) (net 1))
 (via (at 144.78 92.964) (size 0.6858) (drill 0.3302) (layers F.Cu B.Cu) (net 1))
 (segment (start 144.78 91.567) (end 144.78 92.964) (width 0.4064) (layer F.Cu) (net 1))
 (segment (start 144.78 94.615) (end 144.78 96.393) (width 0.4064) (layer F.Cu) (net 1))
 (via (at 135.874 95.488) (size 0.6858) (drill 0.3302) (layers F.Cu B.Cu) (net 1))
 (segment (start 136.398 96.012) (end 135.874 95.488) (width 0.1524) (layer B.Cu) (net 1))
 (segment (start 136.652 96.012) (end 136.398 96.012) (width 0.1524) (layer B.Cu) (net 1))
 (segment (start 135.149 95.488) (end 135.874 95.488) (width 0.1524) (layer F.Cu) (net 1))
 (segment (start 135.874 95.488) (end 136.763 95.488) (width 0.1524) (layer F.Cu) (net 1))
 (via (at 140.335 96.774) (size 0.6858) (drill 0.3302) (layers F.Cu B.Cu) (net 1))
 (segment (start 140.335 96.774) (end 139.065 96.774) (width 0.4064) (layer F.Cu) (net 1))
 (segment (start 140.335 96.393) (end 140.335 96.774) (width 0.4064) (layer F.Cu) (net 1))
 (via (at 138.049 90.424) (size 0.6858) (drill 0.3302) (layers F.Cu B.Cu) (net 1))
 (segment (start 143.3275 94.4805) (end 143.3275 94.668) (width 0.1524) (layer F.Cu) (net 29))
 (segment (start 142.16 93.313) (end 143.3275 94.4805) (width 0.1524) (layer F.Cu) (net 29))
 (segment (start 139.192 93.345) (end 139.224 93.313) (width 0.1524) (layer F.Cu) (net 29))
 (segment (start 139.192 93.867) (end 139.192 93.345) (width 0.1524) (layer F.Cu) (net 29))
 (segment (start 136.524 93.313) (end 139.224 93.313) (width 0.1524) (layer F.Cu) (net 29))
 (segment (start 139.224 93.313) (end 142.16 93.313) (width 0.1524) (layer F.Cu) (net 29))
 (segment (start 138.74 92.513) (end 139.192 92.061) (width 0.1524) (layer F.Cu) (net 28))
 (segment (start 136.524 92.513) (end 138.74 92.513) (width 0.1524) (layer F.Cu) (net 28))
 (segment (start 140.8595 92.061) (end 141.1525 91.768) (width 0.1524) (layer F.Cu) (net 28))
 (segment (start 139.192 92.061) (end 140.8595 92.061) (width 0.1524) (layer F.Cu) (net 28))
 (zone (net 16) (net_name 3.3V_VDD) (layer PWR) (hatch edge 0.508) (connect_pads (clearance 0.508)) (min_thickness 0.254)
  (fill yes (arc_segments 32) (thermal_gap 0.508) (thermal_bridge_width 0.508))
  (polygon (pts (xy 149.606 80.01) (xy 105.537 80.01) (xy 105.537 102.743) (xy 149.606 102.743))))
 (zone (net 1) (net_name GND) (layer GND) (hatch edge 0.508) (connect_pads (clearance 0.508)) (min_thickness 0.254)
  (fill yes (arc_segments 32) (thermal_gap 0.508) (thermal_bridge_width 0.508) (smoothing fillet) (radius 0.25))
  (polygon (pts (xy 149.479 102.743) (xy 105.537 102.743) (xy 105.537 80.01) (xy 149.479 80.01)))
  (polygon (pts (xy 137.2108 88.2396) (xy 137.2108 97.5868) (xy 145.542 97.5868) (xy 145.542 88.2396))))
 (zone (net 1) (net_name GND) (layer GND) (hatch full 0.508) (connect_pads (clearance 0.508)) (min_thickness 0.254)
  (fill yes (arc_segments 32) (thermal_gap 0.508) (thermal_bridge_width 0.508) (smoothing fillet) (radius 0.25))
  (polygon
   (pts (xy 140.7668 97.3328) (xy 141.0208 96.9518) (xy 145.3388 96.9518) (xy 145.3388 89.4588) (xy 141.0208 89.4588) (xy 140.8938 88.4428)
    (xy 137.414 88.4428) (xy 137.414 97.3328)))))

